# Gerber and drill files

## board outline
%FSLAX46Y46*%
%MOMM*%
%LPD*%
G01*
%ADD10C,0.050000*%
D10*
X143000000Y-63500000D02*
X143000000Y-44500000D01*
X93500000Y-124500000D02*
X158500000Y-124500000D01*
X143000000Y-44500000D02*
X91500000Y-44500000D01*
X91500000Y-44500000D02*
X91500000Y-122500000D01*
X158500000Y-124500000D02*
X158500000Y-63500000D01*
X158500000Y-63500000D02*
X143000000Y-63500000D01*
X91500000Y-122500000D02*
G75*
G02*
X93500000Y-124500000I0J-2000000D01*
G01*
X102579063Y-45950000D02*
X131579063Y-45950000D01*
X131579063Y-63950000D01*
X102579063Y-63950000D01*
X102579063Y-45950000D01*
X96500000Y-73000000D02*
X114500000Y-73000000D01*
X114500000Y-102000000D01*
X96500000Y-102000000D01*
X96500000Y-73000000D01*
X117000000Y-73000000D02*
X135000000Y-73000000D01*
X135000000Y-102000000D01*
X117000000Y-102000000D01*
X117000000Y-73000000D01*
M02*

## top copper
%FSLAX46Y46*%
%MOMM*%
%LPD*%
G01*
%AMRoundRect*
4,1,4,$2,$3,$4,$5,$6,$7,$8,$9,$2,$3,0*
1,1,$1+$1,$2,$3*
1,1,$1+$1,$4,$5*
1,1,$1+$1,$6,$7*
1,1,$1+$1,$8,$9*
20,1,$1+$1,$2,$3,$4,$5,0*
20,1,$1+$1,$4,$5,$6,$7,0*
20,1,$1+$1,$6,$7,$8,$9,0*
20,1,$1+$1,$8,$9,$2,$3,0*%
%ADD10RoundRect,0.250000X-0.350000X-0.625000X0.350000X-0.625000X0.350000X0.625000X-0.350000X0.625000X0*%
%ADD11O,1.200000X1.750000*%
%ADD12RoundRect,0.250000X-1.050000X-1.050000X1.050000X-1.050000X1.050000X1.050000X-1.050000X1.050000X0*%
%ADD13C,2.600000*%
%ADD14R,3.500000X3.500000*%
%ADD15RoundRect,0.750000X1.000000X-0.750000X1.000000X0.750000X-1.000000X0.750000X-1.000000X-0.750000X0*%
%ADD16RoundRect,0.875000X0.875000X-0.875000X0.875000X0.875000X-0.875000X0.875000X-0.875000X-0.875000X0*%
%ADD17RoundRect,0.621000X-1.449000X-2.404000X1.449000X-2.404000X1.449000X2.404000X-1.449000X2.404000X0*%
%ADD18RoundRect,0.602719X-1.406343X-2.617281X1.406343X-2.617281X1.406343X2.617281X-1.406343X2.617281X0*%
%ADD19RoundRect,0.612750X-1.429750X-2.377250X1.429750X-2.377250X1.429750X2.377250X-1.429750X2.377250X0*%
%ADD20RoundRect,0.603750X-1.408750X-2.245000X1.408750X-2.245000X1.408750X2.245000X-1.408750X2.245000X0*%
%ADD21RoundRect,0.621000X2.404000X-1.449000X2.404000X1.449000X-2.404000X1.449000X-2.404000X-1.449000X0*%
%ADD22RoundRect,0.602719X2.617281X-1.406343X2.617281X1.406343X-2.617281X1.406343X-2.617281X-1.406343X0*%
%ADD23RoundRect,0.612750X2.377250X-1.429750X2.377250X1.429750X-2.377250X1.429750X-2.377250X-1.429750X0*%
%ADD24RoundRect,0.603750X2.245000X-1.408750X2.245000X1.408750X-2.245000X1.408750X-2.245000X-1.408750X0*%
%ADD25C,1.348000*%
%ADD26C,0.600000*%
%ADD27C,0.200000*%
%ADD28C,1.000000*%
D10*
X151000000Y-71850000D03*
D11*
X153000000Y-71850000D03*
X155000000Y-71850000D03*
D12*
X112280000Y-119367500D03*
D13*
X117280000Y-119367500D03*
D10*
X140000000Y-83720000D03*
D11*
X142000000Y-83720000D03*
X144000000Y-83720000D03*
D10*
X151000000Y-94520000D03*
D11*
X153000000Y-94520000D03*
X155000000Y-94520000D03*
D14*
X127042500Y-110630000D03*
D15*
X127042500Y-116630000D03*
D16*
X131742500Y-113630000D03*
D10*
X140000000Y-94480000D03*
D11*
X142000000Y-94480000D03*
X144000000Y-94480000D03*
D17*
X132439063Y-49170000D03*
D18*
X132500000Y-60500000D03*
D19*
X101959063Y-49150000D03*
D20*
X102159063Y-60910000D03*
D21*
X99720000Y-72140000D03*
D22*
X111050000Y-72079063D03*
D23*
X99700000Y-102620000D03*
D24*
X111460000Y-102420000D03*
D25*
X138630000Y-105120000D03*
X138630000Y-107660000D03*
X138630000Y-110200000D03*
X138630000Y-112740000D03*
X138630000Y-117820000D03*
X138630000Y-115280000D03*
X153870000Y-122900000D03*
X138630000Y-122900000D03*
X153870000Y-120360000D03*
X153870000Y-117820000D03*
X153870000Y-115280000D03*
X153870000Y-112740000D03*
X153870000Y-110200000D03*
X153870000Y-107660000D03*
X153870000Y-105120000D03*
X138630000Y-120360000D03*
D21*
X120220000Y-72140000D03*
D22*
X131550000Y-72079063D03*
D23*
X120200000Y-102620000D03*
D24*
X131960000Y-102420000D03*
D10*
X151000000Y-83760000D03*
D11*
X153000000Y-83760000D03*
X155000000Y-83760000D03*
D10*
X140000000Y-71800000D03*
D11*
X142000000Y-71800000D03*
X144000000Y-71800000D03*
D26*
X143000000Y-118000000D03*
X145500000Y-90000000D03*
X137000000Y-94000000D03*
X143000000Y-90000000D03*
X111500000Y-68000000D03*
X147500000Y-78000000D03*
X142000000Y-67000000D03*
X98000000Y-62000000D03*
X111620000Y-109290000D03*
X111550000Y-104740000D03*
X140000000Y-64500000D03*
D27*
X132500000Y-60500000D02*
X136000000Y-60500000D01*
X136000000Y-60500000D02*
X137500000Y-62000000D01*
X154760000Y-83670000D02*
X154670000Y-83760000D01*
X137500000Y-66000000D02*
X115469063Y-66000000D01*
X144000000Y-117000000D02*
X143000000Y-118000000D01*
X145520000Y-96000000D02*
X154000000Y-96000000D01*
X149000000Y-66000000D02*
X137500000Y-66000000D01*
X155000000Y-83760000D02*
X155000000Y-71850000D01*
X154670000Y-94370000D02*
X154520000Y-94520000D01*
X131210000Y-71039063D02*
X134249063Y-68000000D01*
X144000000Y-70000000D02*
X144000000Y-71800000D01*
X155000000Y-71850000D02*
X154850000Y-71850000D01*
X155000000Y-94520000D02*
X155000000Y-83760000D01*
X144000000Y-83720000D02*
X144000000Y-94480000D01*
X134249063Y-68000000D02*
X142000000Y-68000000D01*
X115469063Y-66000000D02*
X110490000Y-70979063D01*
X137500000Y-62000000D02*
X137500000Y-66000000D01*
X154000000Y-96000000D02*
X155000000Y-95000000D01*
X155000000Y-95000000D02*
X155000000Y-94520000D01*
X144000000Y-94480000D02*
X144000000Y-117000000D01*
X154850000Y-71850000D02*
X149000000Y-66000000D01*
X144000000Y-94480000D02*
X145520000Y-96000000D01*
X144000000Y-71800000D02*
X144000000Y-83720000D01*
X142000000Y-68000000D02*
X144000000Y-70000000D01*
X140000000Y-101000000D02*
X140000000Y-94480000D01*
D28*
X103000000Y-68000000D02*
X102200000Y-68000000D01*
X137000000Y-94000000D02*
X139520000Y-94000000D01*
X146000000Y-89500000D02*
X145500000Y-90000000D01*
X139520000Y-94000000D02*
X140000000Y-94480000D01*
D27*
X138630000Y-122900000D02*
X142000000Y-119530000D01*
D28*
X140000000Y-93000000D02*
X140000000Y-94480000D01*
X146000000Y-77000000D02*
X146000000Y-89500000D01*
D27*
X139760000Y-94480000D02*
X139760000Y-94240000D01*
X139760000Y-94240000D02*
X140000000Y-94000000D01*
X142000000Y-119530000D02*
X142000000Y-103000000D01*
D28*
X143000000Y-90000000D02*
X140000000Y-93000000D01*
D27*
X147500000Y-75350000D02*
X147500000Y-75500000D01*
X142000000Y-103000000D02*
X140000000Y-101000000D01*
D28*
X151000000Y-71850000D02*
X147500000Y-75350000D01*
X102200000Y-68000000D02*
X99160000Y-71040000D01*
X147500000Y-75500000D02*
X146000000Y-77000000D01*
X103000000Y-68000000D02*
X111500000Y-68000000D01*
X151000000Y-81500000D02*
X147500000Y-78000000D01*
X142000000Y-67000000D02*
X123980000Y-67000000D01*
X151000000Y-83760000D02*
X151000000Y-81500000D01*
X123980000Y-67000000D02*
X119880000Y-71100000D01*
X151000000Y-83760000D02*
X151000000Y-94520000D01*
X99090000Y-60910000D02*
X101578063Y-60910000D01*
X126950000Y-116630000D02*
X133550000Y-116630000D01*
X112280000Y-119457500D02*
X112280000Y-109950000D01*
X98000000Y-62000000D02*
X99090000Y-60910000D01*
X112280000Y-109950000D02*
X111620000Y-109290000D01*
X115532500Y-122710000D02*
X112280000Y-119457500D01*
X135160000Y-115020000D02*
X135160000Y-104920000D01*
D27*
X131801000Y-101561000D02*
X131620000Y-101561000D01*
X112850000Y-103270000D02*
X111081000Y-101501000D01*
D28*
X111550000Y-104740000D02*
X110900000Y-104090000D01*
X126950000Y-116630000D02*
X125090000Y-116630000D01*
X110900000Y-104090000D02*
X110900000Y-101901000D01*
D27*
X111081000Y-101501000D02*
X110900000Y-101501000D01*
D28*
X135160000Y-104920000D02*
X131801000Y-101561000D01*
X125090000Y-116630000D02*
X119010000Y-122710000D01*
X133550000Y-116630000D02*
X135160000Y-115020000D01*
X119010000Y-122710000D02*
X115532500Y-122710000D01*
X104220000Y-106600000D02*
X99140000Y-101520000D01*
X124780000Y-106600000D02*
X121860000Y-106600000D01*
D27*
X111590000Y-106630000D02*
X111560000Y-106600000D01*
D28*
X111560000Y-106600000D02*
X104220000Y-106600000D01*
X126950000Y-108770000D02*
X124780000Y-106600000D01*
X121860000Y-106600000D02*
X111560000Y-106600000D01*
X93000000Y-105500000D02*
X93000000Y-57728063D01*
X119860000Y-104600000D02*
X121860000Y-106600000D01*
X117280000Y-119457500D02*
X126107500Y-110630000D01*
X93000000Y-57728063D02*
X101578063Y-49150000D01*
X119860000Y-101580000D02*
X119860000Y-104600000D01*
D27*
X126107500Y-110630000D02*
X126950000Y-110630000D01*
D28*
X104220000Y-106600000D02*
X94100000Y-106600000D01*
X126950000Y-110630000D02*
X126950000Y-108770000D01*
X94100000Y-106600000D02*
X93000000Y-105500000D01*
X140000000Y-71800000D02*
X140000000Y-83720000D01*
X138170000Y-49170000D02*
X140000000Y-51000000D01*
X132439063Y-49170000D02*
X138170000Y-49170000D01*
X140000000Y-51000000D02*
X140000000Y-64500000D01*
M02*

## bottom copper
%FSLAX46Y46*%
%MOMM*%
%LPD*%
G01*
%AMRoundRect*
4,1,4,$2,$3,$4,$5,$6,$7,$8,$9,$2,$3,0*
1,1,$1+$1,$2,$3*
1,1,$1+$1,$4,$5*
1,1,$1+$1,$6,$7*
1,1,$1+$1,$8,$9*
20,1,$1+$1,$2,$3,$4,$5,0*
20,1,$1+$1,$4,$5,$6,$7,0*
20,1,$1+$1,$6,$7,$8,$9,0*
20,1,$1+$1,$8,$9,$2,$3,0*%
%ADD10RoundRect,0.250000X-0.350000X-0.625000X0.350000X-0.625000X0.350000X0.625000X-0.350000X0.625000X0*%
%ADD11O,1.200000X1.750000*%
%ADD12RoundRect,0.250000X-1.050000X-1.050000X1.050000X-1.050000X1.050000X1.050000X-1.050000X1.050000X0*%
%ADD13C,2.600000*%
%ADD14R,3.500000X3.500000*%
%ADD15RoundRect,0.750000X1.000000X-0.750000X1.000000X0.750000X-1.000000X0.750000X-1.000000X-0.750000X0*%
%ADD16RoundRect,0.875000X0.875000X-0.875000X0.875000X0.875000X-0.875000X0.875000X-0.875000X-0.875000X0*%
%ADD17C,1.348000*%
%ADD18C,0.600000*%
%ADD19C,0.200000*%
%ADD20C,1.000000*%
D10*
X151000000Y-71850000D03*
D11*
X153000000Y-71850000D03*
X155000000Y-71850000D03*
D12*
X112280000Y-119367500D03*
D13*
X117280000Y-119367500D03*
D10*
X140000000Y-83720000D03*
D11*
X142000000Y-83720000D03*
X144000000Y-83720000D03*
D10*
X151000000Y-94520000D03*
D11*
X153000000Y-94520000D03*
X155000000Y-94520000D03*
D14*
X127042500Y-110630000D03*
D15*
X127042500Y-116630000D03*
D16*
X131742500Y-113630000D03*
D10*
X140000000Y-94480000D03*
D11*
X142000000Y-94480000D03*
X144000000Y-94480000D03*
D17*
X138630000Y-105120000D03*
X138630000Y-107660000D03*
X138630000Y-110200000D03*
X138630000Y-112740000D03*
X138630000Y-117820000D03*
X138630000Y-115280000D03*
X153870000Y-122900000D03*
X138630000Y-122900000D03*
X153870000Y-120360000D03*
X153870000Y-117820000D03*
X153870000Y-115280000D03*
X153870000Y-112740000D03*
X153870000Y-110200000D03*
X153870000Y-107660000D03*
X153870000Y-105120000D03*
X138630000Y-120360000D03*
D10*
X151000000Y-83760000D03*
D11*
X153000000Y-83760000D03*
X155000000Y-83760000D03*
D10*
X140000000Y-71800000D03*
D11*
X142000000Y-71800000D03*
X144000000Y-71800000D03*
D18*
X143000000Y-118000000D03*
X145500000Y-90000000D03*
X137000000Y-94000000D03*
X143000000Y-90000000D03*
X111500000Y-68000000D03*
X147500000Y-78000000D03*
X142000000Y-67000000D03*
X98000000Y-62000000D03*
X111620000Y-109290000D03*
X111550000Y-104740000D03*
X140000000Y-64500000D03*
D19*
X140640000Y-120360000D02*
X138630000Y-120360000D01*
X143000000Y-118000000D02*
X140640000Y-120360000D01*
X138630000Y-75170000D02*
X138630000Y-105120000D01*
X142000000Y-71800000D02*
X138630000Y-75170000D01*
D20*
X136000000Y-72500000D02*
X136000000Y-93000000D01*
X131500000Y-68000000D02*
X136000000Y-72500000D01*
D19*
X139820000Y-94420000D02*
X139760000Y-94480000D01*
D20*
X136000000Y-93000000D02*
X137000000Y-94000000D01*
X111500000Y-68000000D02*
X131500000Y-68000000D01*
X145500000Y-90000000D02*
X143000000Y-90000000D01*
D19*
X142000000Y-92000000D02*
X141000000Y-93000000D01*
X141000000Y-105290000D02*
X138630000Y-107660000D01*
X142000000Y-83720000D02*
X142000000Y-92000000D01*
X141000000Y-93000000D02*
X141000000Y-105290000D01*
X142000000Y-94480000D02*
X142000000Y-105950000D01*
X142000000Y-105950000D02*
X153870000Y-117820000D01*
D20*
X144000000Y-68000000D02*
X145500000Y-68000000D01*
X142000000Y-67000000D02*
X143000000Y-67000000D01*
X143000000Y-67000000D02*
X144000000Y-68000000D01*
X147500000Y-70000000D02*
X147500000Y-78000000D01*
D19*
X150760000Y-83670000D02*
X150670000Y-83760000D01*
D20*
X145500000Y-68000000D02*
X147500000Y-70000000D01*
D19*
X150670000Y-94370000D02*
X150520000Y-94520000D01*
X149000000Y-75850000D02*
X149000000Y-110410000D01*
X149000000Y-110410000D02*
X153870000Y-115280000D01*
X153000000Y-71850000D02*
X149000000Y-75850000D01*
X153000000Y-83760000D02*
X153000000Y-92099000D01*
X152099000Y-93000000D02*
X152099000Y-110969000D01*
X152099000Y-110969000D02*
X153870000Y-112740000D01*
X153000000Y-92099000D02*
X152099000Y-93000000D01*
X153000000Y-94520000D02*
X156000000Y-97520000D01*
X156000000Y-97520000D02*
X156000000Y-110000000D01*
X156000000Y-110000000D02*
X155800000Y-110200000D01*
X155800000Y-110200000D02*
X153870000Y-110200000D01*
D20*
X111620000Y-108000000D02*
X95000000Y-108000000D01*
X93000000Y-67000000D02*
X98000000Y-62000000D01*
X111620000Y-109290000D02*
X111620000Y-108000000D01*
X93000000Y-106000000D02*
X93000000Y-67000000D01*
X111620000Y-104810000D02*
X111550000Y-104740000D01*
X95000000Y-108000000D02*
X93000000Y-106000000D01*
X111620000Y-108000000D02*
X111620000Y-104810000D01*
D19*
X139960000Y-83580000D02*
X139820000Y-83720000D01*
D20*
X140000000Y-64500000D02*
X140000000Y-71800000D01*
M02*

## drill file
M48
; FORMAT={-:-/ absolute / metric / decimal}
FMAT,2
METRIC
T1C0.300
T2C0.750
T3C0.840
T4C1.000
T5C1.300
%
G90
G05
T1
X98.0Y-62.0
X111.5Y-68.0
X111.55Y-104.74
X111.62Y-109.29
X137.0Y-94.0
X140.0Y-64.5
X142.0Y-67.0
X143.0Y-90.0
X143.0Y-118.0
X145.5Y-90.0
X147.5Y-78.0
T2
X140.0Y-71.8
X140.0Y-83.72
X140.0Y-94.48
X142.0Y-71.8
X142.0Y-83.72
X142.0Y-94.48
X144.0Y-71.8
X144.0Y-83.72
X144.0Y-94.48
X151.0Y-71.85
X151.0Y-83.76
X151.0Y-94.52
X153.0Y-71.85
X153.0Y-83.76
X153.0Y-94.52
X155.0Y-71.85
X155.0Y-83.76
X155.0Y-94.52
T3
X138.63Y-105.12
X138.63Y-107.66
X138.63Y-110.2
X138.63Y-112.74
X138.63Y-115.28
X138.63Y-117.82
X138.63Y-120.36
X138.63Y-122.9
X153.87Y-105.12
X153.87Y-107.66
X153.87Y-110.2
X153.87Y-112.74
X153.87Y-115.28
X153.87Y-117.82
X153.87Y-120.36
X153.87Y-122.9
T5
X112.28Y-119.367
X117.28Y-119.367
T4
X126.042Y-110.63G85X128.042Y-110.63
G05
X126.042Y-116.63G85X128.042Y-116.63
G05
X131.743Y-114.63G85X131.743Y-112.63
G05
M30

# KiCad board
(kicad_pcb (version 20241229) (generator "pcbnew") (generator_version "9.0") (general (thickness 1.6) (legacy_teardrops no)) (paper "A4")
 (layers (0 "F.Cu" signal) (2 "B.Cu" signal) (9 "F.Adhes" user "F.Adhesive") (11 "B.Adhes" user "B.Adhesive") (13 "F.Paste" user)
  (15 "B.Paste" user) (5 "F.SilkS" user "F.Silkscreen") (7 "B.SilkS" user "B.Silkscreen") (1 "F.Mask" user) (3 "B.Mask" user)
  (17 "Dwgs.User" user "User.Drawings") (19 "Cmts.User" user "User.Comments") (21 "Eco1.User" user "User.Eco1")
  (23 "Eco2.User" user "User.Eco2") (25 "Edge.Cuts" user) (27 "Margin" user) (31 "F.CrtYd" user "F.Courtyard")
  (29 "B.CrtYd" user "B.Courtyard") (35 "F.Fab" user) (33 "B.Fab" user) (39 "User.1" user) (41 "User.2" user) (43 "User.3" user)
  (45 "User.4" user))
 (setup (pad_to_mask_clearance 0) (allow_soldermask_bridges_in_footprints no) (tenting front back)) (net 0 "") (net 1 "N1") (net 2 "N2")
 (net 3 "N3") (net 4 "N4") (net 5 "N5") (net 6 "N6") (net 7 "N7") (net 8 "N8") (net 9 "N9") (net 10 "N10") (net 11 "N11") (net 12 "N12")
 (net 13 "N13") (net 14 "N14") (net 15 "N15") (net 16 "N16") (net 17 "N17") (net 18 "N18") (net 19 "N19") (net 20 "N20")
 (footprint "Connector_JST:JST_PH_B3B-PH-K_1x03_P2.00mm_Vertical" (layer "F.Cu") (at 151 71.85)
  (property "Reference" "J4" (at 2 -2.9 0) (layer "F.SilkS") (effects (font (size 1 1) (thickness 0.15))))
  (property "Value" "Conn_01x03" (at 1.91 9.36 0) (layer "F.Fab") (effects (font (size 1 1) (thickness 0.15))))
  (pad "1" thru_hole roundrect (at 0 0) (size 1.2 1.75) (drill 0.75) (layers "*.Cu" "*.Mask") (remove_unused_layers no)
   (roundrect_rratio 0.208333) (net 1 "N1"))
  (pad "2" thru_hole oval (at 2 0) (size 1.2 1.75) (drill 0.75) (layers "*.Cu" "*.Mask") (remove_unused_layers no) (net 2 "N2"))
  (pad "3" thru_hole oval (at 4 0) (size 1.2 1.75) (drill 0.75) (layers "*.Cu" "*.Mask") (remove_unused_layers no) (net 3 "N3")))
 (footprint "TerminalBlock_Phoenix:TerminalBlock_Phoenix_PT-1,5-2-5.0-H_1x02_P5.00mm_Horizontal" (layer "F.Cu") (at 112.28 119.3675)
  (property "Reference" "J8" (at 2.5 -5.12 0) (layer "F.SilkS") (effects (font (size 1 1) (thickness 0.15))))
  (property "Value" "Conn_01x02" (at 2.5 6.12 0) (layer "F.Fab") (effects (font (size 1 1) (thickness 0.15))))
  (pad "1" thru_hole roundrect (at 0 0) (size 2.6 2.6) (drill 1.3) (layers "*.Cu" "*.Mask") (remove_unused_layers no)
   (roundrect_rratio 0.096154) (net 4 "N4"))
  (pad "2" thru_hole circle (at 5 0) (size 2.6 2.6) (drill 1.3) (layers "*.Cu" "*.Mask") (remove_unused_layers no) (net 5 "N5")))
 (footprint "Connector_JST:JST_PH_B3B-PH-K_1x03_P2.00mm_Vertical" (layer "F.Cu") (at 140 83.72)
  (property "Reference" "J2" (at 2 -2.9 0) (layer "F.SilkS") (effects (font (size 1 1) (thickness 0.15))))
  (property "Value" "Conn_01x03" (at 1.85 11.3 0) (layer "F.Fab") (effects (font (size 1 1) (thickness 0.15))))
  (pad "1" thru_hole roundrect (at 0 0) (size 1.2 1.75) (drill 0.75) (layers "*.Cu" "*.Mask") (remove_unused_layers no)
   (roundrect_rratio 0.208333) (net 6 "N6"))
  (pad "2" thru_hole oval (at 2 0) (size 1.2 1.75) (drill 0.75) (layers "*.Cu" "*.Mask") (remove_unused_layers no) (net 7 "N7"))
  (pad "3" thru_hole oval (at 4 0) (size 1.2 1.75) (drill 0.75) (layers "*.Cu" "*.Mask") (remove_unused_layers no) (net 3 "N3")))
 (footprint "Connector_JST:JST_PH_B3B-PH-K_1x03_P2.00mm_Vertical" (layer "F.Cu") (at 151 94.52)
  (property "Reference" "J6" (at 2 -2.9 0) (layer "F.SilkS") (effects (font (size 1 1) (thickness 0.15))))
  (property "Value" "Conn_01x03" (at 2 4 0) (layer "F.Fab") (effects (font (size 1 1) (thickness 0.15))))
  (pad "1" thru_hole roundrect (at 0 0) (size 1.2 1.75) (drill 0.75) (layers "*.Cu" "*.Mask") (remove_unused_layers no)
   (roundrect_rratio 0.208333) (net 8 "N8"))
  (pad "2" thru_hole oval (at 2 0) (size 1.2 1.75) (drill 0.75) (layers "*.Cu" "*.Mask") (remove_unused_layers no) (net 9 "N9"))
  (pad "3" thru_hole oval (at 4 0) (size 1.2 1.75) (drill 0.75) (layers "*.Cu" "*.Mask") (remove_unused_layers no) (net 3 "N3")))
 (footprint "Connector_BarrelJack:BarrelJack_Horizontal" (layer "F.Cu") (at 127.0425 110.63 90)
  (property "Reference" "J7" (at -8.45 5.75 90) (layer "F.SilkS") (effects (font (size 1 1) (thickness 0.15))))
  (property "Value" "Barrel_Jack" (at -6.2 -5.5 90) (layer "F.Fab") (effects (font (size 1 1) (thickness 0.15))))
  (pad "1" thru_hole rect (at 0 0 90) (size 3.5 3.5) (drill oval 1 3) (layers "*.Cu" "*.Mask") (remove_unused_layers no) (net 5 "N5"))
  (pad "2" thru_hole roundrect (at -6 0 90) (size 3 3.5) (drill oval 1 3) (layers "*.Cu" "*.Mask") (remove_unused_layers no)
   (roundrect_rratio 0.25) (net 4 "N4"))
  (pad "3" thru_hole roundrect (at -3 4.7 90) (size 3.5 3.5) (drill oval 3 1) (layers "*.Cu" "*.Mask") (remove_unused_layers no)
   (roundrect_rratio 0.25)))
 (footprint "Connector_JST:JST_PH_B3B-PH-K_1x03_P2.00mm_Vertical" (layer "F.Cu") (at 140 94.48)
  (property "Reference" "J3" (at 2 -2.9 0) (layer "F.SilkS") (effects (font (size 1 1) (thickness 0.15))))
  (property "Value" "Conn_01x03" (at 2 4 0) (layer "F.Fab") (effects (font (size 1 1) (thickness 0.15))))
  (pad "1" thru_hole roundrect (at 0 0) (size 1.2 1.75) (drill 0.75) (layers "*.Cu" "*.Mask") (remove_unused_layers no)
   (roundrect_rratio 0.208333) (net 1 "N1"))
  (pad "2" thru_hole oval (at 2 0) (size 1.2 1.75) (drill 0.75) (layers "*.Cu" "*.Mask") (remove_unused_layers no) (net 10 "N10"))
  (pad "3" thru_hole oval (at 4 0) (size 1.2 1.75) (drill 0.75) (layers "*.Cu" "*.Mask") (remove_unused_layers no) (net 3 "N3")))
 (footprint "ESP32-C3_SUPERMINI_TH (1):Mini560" (layer "F.Cu") (at 116.579063 52.95)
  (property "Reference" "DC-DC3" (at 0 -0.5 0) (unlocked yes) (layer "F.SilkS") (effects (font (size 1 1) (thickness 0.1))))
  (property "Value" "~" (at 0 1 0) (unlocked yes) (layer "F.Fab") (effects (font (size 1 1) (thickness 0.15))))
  (fp_rect (start -14 -7) (end 15 11) (stroke (width 0.05) (type default)) (fill no) (layer "Edge.Cuts"))
  (pad "1" smd roundrect (at 15.86 -3.78) (size 4.14 6.05) (layers "F.Cu" "F.Mask" "F.Paste") (roundrect_rratio 0.15) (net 6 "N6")
   (thermal_bridge_angle 45))
  (pad "2" smd roundrect (at 15.920937 7.55) (size 4.018125 6.44) (layers "F.Cu" "F.Mask" "F.Paste") (roundrect_rratio 0.15) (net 3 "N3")
   (thermal_bridge_angle 45))
  (pad "3" smd roundrect (at -14.62 -3.8) (size 4.085 5.98) (layers "F.Cu" "F.Mask" "F.Paste") (roundrect_rratio 0.15) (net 5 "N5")
   (thermal_bridge_angle 45))
  (pad "4" smd roundrect (at -14.42 7.96) (size 4.025 5.6975) (layers "F.Cu" "F.Mask" "F.Paste") (roundrect_rratio 0.15) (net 4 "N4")
   (thermal_bridge_angle 45)))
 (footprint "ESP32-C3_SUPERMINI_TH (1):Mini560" (layer "F.Cu") (at 103.5 88 90)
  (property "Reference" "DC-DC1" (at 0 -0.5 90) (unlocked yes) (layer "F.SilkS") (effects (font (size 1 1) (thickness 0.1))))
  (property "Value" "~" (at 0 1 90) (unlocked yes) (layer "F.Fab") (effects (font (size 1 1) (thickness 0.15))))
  (fp_rect (start -14 -7) (end 15 11) (stroke (width 0.05) (type default)) (fill no) (layer "Edge.Cuts"))
  (pad "1" smd roundrect (at 15.86 -3.78 90) (size 4.14 6.05) (layers "F.Cu" "F.Mask" "F.Paste") (roundrect_rratio 0.15) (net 1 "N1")
   (thermal_bridge_angle 45))
  (pad "2" smd roundrect (at 15.920937 7.55 90) (size 4.018125 6.44) (layers "F.Cu" "F.Mask" "F.Paste") (roundrect_rratio 0.15) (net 3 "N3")
   (thermal_bridge_angle 45))
  (pad "3" smd roundrect (at -14.62 -3.8 90) (size 4.085 5.98) (layers "F.Cu" "F.Mask" "F.Paste") (roundrect_rratio 0.15) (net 5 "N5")
   (thermal_bridge_angle 45))
  (pad "4" smd roundrect (at -14.42 7.96 90) (size 4.025 5.6975) (layers "F.Cu" "F.Mask" "F.Paste") (roundrect_rratio 0.15) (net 4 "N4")
   (thermal_bridge_angle 45)))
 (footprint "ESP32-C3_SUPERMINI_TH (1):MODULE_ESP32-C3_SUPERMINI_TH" (layer "F.Cu") (at 146.25 113 180)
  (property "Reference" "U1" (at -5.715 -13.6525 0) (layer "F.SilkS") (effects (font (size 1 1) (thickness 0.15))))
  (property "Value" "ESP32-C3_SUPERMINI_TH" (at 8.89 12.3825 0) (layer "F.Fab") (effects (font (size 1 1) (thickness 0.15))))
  (pad "0" thru_hole circle (at 7.62 7.88 180) (size 1.348 1.348) (drill 0.84) (layers "*.Cu" "*.Mask") (remove_unused_layers no)
   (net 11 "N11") (solder_mask_margin 0.102))
  (pad "1" thru_hole circle (at 7.62 5.34 180) (size 1.348 1.348) (drill 0.84) (layers "*.Cu" "*.Mask") (remove_unused_layers no)
   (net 7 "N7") (solder_mask_margin 0.102))
  (pad "2" thru_hole circle (at 7.62 2.8 180) (size 1.348 1.348) (drill 0.84) (layers "*.Cu" "*.Mask") (remove_unused_layers no)
   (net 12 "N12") (solder_mask_margin 0.102))
  (pad "3" thru_hole circle (at 7.62 0.26 180) (size 1.348 1.348) (drill 0.84) (layers "*.Cu" "*.Mask") (remove_unused_layers no)
   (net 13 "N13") (solder_mask_margin 0.102))
  (pad "3.3" thru_hole circle (at 7.62 -4.82 180) (size 1.348 1.348) (drill 0.84) (layers "*.Cu" "*.Mask") (remove_unused_layers no)
   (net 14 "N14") (solder_mask_margin 0.102))
  (pad "4" thru_hole circle (at 7.62 -2.28 180) (size 1.348 1.348) (drill 0.84) (layers "*.Cu" "*.Mask") (remove_unused_layers no)
   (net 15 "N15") (solder_mask_margin 0.102))
  (pad "5" thru_hole circle (at -7.62 -9.9 180) (size 1.348 1.348) (drill 0.84) (layers "*.Cu" "*.Mask") (remove_unused_layers no)
   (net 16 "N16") (solder_mask_margin 0.102))
  (pad "5V" thru_hole circle (at 7.62 -9.9 180) (size 1.348 1.348) (drill 0.84) (layers "*.Cu" "*.Mask") (remove_unused_layers no)
   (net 1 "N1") (solder_mask_margin 0.102))
  (pad "6" thru_hole circle (at -7.62 -7.36 180) (size 1.348 1.348) (drill 0.84) (layers "*.Cu" "*.Mask") (remove_unused_layers no)
   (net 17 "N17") (solder_mask_margin 0.102))
  (pad "7" thru_hole circle (at -7.62 -4.82 180) (size 1.348 1.348) (drill 0.84) (layers "*.Cu" "*.Mask") (remove_unused_layers no)
   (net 10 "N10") (solder_mask_margin 0.102))
  (pad "8" thru_hole circle (at -7.62 -2.28 180) (size 1.348 1.348) (drill 0.84) (layers "*.Cu" "*.Mask") (remove_unused_layers no)
   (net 2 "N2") (solder_mask_margin 0.102))
  (pad "9" thru_hole circle (at -7.62 0.26 180) (size 1.348 1.348) (drill 0.84) (layers "*.Cu" "*.Mask") (remove_unused_layers no)
   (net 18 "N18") (solder_mask_margin 0.102))
  (pad "10" thru_hole circle (at -7.62 2.8 180) (size 1.348 1.348) (drill 0.84) (layers "*.Cu" "*.Mask") (remove_unused_layers no)
   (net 9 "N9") (solder_mask_margin 0.102))
  (pad "20" thru_hole circle (at -7.62 5.34 180) (size 1.348 1.348) (drill 0.84) (layers "*.Cu" "*.Mask") (remove_unused_layers no)
   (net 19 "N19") (solder_mask_margin 0.102))
  (pad "21" thru_hole circle (at -7.62 7.88 180) (size 1.348 1.348) (drill 0.84) (layers "*.Cu" "*.Mask") (remove_unused_layers no)
   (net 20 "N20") (solder_mask_margin 0.102))
  (pad "G" thru_hole circle (at 7.62 -7.36 180) (size 1.348 1.348) (drill 0.84) (layers "*.Cu" "*.Mask") (remove_unused_layers no)
   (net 3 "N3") (solder_mask_margin 0.102)))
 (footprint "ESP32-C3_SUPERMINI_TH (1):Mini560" (layer "F.Cu") (at 124 88 90)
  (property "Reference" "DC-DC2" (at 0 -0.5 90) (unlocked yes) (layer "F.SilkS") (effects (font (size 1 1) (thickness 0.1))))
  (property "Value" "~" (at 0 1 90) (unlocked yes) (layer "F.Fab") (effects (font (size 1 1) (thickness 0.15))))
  (fp_rect (start -14 -7) (end 15 11) (stroke (width 0.05) (type default)) (fill no) (layer "Edge.Cuts"))
  (pad "1" smd roundrect (at 15.86 -3.78 90) (size 4.14 6.05) (layers "F.Cu" "F.Mask" "F.Paste") (roundrect_rratio 0.15) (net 8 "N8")
   (thermal_bridge_angle 45))
  (pad "2" smd roundrect (at 15.920937 7.55 90) (size 4.018125 6.44) (layers "F.Cu" "F.Mask" "F.Paste") (roundrect_rratio 0.15) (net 3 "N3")
   (thermal_bridge_angle 45))
  (pad "3" smd roundrect (at -14.62 -3.8 90) (size 4.085 5.98) (layers "F.Cu" "F.Mask" "F.Paste") (roundrect_rratio 0.15) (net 5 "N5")
   (thermal_bridge_angle 45))
  (pad "4" smd roundrect (at -14.42 7.96 90) (size 4.025 5.6975) (layers "F.Cu" "F.Mask" "F.Paste") (roundrect_rratio 0.15) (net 4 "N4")
   (thermal_bridge_angle 45)))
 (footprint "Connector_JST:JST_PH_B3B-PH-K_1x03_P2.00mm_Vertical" (layer "F.Cu") (at 151 83.76)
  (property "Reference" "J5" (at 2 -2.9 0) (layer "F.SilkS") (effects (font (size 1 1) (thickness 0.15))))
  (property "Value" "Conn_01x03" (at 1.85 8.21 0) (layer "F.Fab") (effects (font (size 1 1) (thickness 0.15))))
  (pad "1" thru_hole roundrect (at 0 0) (size 1.2 1.75) (drill 0.75) (layers "*.Cu" "*.Mask") (remove_unused_layers no)
   (roundrect_rratio 0.208333) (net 8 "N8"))
  (pad "2" thru_hole oval (at 2 0) (size 1.2 1.75) (drill 0.75) (layers "*.Cu" "*.Mask") (remove_unused_layers no) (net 18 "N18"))
  (pad "3" thru_hole oval (at 4 0) (size 1.2 1.75) (drill 0.75) (layers "*.Cu" "*.Mask") (remove_unused_layers no) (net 3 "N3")))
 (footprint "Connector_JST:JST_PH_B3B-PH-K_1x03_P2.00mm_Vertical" (layer "F.Cu") (at 140 71.8)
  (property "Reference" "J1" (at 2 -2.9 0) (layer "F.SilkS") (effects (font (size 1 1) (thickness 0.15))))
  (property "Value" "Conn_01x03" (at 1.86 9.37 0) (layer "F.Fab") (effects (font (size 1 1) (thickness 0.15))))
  (pad "1" thru_hole roundrect (at 0 0) (size 1.2 1.75) (drill 0.75) (layers "*.Cu" "*.Mask") (remove_unused_layers no)
   (roundrect_rratio 0.208333) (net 6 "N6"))
  (pad "2" thru_hole oval (at 2 0) (size 1.2 1.75) (drill 0.75) (layers "*.Cu" "*.Mask") (remove_unused_layers no) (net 11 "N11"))
  (pad "3" thru_hole oval (at 4 0) (size 1.2 1.75) (drill 0.75) (layers "*.Cu" "*.Mask") (remove_unused_layers no) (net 3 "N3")))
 (gr_line (start 143 63.5) (end 143 44.5) (stroke (width 0.05) (type default)) (layer "Edge.Cuts"))
 (gr_line (start 93.5 124.5) (end 158.5 124.5) (stroke (width 0.05) (type default)) (layer "Edge.Cuts"))
 (gr_line (start 143 44.5) (end 91.5 44.5) (stroke (width 0.05) (type default)) (layer "Edge.Cuts"))
 (gr_line (start 91.5 44.5) (end 91.5 122.5) (stroke (width 0.05) (type default)) (layer "Edge.Cuts"))
 (gr_line (start 158.5 124.5) (end 158.5 63.5) (stroke (width 0.05) (type default)) (layer "Edge.Cuts"))
 (gr_line (start 158.5 63.5) (end 143 63.5) (stroke (width 0.05) (type default)) (layer "Edge.Cuts"))
 (gr_arc (start 91.5 122.5) (mid 92.914214 123.085786) (end 93.5 124.5) (stroke (width 0.05) (type default)) (layer "Edge.Cuts"))
 (segment (start 132.5 60.5) (end 136 60.5) (width 0.2) (layer "F.Cu") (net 3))
 (segment (start 136 60.5) (end 137.5 62) (width 0.2) (layer "F.Cu") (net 3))
 (segment (start 154.76 83.67) (end 154.67 83.76) (width 0.2) (layer "F.Cu") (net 3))
 (segment (start 137.5 66) (end 115.469063 66) (width 0.2) (layer "F.Cu") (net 3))
 (segment (start 144 117) (end 143 118) (width 0.2) (layer "F.Cu") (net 3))
 (segment (start 145.52 96) (end 154 96) (width 0.2) (layer "F.Cu") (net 3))
 (segment (start 149 66) (end 137.5 66) (width 0.2) (layer "F.Cu") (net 3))
 (segment (start 155 83.76) (end 155 71.85) (width 0.2) (layer "F.Cu") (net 3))
 (segment (start 154.67 94.37) (end 154.52 94.52) (width 0.2) (layer "F.Cu") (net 3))
 (segment (start 131.21 71.039063) (end 134.249063 68) (width 0.2) (layer "F.Cu") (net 3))
 (segment (start 144 70) (end 144 71.8) (width 0.2) (layer "F.Cu") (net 3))
 (segment (start 155 71.85) (end 154.85 71.85) (width 0.2) (layer "F.Cu") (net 3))
 (segment (start 155 94.52) (end 155 83.76) (width 0.2) (layer "F.Cu") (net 3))
 (segment (start 144 83.72) (end 144 94.48) (width 0.2) (layer "F.Cu") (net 3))
 (segment (start 134.249063 68) (end 142 68) (width 0.2) (layer "F.Cu") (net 3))
 (segment (start 115.469063 66) (end 110.49 70.979063) (width 0.2) (layer "F.Cu") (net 3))
 (segment (start 137.5 62) (end 137.5 66) (width 0.2) (layer "F.Cu") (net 3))
 (segment (start 154 96) (end 155 95) (width 0.2) (layer "F.Cu") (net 3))
 (segment (start 155 95) (end 155 94.52) (width 0.2) (layer "F.Cu") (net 3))
 (segment (start 144 94.48) (end 144 117) (width 0.2) (layer "F.Cu") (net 3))
 (segment (start 154.85 71.85) (end 149 66) (width 0.2) (layer "F.Cu") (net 3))
 (segment (start 144 94.48) (end 145.52 96) (width 0.2) (layer "F.Cu") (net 3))
 (segment (start 144 71.8) (end 144 83.72) (width 0.2) (layer "F.Cu") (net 3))
 (segment (start 142 68) (end 144 70) (width 0.2) (layer "F.Cu") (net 3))
 (via (at 143 118) (size 0.6) (drill 0.3) (layers "F.Cu" "B.Cu") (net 3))
 (segment (start 140.64 120.36) (end 138.63 120.36) (width 0.2) (layer "B.Cu") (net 3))
 (segment (start 143 118) (end 140.64 120.36) (width 0.2) (layer "B.Cu") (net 3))
 (segment (start 138.63 75.17) (end 138.63 105.12) (width 0.2) (layer "B.Cu") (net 11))
 (segment (start 142 71.8) (end 138.63 75.17) (width 0.2) (layer "B.Cu") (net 11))
 (segment (start 140 101) (end 140 94.48) (width 0.2) (layer "F.Cu") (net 1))
 (segment (start 103 68) (end 102.2 68) (width 1) (layer "F.Cu") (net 1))
 (segment (start 137 94) (end 139.52 94) (width 1) (layer "F.Cu") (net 1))
 (segment (start 146 89.5) (end 145.5 90) (width 1) (layer "F.Cu") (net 1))
 (segment (start 139.52 94) (end 140 94.48) (width 1) (layer "F.Cu") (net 1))
 (segment (start 138.63 122.9) (end 142 119.53) (width 0.2) (layer "F.Cu") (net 1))
 (segment (start 140 93) (end 140 94.48) (width 1) (layer "F.Cu") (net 1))
 (segment (start 146 77) (end 146 89.5) (width 1) (layer "F.Cu") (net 1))
 (segment (start 139.76 94.48) (end 139.76 94.24) (width 0.2) (layer "F.Cu") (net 1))
 (segment (start 139.76 94.24) (end 140 94) (width 0.2) (layer "F.Cu") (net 1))
 (segment (start 142 119.53) (end 142 103) (width 0.2) (layer "F.Cu") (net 1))
 (segment (start 143 90) (end 140 93) (width 1) (layer "F.Cu") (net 1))
 (segment (start 147.5 75.35) (end 147.5 75.5) (width 0.2) (layer "F.Cu") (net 1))
 (segment (start 142 103) (end 140 101) (width 0.2) (layer "F.Cu") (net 1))
 (segment (start 151 71.85) (end 147.5 75.35) (width 1) (layer "F.Cu") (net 1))
 (segment (start 102.2 68) (end 99.16 71.04) (width 1) (layer "F.Cu") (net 1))
 (segment (start 147.5 75.5) (end 146 77) (width 1) (layer "F.Cu") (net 1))
 (segment (start 103 68) (end 111.5 68) (width 1) (layer "F.Cu") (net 1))
 (via (at 145.5 90) (size 0.6) (drill 0.3) (layers "F.Cu" "B.Cu") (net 1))
 (via (at 137 94) (size 0.6) (drill 0.3) (layers "F.Cu" "B.Cu") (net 1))
 (via (at 143 90) (size 0.6) (drill 0.3) (layers "F.Cu" "B.Cu") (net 1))
 (via (at 111.5 68) (size 0.6) (drill 0.3) (layers "F.Cu" "B.Cu") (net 1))
 (segment (start 136 72.5) (end 136 93) (width 1) (layer "B.Cu") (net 1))
 (segment (start 131.5 68) (end 136 72.5) (width 1) (layer "B.Cu") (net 1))
 (segment (start 139.82 94.42) (end 139.76 94.48) (width 0.2) (layer "B.Cu") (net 1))
 (segment (start 136 93) (end 137 94) (width 1) (layer "B.Cu") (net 1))
 (segment (start 111.5 68) (end 131.5 68) (width 1) (layer "B.Cu") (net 1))
 (segment (start 145.5 90) (end 143 90) (width 1) (layer "B.Cu") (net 1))
 (segment (start 142 92) (end 141 93) (width 0.2) (layer "B.Cu") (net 7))
 (segment (start 141 105.29) (end 138.63 107.66) (width 0.2) (layer "B.Cu") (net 7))
 (segment (start 142 83.72) (end 142 92) (width 0.2) (layer "B.Cu") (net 7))
 (segment (start 141 93) (end 141 105.29) (width 0.2) (layer "B.Cu") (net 7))
 (segment (start 142 94.48) (end 142 105.95) (width 0.2) (layer "B.Cu") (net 10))
 (segment (start 142 105.95) (end 153.87 117.82) (width 0.2) (layer "B.Cu") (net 10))
 (segment (start 151 81.5) (end 147.5 78) (width 1) (layer "F.Cu") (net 8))
 (segment (start 142 67) (end 123.98 67) (width 1) (layer "F.Cu") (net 8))
 (segment (start 151 83.76) (end 151 81.5) (width 1) (layer "F.Cu") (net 8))
 (segment (start 123.98 67) (end 119.88 71.1) (width 1) (layer "F.Cu") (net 8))
 (segment (start 151 83.76) (end 151 94.52) (width 1) (layer "F.Cu") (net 8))
 (via (at 147.5 78) (size 0.6) (drill 0.3) (layers "F.Cu" "B.Cu") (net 8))
 (via (at 142 67) (size 0.6) (drill 0.3) (layers "F.Cu" "B.Cu") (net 8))
 (segment (start 144 68) (end 145.5 68) (width 1) (layer "B.Cu") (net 8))
 (segment (start 142 67) (end 143 67) (width 1) (layer "B.Cu") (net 8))
 (segment (start 143 67) (end 144 68) (width 1) (layer "B.Cu") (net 8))
 (segment (start 147.5 70) (end 147.5 78) (width 1) (layer "B.Cu") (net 8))
 (segment (start 150.76 83.67) (end 150.67 83.76) (width 0.2) (layer "B.Cu") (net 8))
 (segment (start 145.5 68) (end 147.5 70) (width 1) (layer "B.Cu") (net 8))
 (segment (start 150.67 94.37) (end 150.52 94.52) (width 0.2) (layer "B.Cu") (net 8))
 (segment (start 149 75.85) (end 149 110.41) (width 0.2) (layer "B.Cu") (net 2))
 (segment (start 149 110.41) (end 153.87 115.28) (width 0.2) (layer "B.Cu") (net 2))
 (segment (start 153 71.85) (end 149 75.85) (width 0.2) (layer "B.Cu") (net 2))
 (segment (start 153 83.76) (end 153 92.099) (width 0.2) (layer "B.Cu") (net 18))
 (segment (start 152.099 93) (end 152.099 110.969) (width 0.2) (layer "B.Cu") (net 18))
 (segment (start 152.099 110.969) (end 153.87 112.74) (width 0.2) (layer "B.Cu") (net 18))
 (segment (start 153 92.099) (end 152.099 93) (width 0.2) (layer "B.Cu") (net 18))
 (segment (start 153 94.52) (end 156 97.52) (width 0.2) (layer "B.Cu") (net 9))
 (segment (start 156 97.52) (end 156 110) (width 0.2) (layer "B.Cu") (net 9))
 (segment (start 156 110) (end 155.8 110.2) (width 0.2) (layer "B.Cu") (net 9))
 (segment (start 155.8 110.2) (end 153.87 110.2) (width 0.2) (layer "B.Cu") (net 9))
 (segment (start 99.09 60.91) (end 101.578063 60.91) (width 1) (layer "F.Cu") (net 4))
 (segment (start 126.95 116.63) (end 133.55 116.63) (width 1) (layer "F.Cu") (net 4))
 (segment (start 112.28 119.4575) (end 112.28 109.95) (width 1) (layer "F.Cu") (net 4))
 (segment (start 98 62) (end 99.09 60.91) (width 1) (layer "F.Cu") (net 4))
 (segment (start 112.28 109.95) (end 111.62 109.29) (width 1) (layer "F.Cu") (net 4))
 (segment (start 115.5325 122.71) (end 112.28 119.4575) (width 1) (layer "F.Cu") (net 4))
 (segment (start 135.16 115.02) (end 135.16 104.92) (width 1) (layer "F.Cu") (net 4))
 (segment (start 131.801 101.561) (end 131.62 101.561) (width 0.2) (layer "F.Cu") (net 4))
 (segment (start 112.85 103.27) (end 111.081 101.501) (width 0.2) (layer "F.Cu") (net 4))
 (segment (start 111.55 104.74) (end 110.9 104.09) (width 1) (layer "F.Cu") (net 4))
 (segment (start 126.95 116.63) (end 125.09 116.63) (width 1) (layer "F.Cu") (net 4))
 (segment (start 110.9 104.09) (end 110.9 101.901) (width 1) (layer "F.Cu") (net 4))
 (segment (start 111.081 101.501) (end 110.9 101.501) (width 0.2) (layer "F.Cu") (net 4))
 (segment (start 135.16 104.92) (end 131.801 101.561) (width 1) (layer "F.Cu") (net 4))
 (segment (start 125.09 116.63) (end 119.01 122.71) (width 1) (layer "F.Cu") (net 4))
 (segment (start 133.55 116.63) (end 135.16 115.02) (width 1) (layer "F.Cu") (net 4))
 (segment (start 119.01 122.71) (end 115.5325 122.71) (width 1) (layer "F.Cu") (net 4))
 (via (at 98 62) (size 0.6) (drill 0.3) (layers "F.Cu" "B.Cu") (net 4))
 (via (at 111.62 109.29) (size 0.6) (drill 0.3) (layers "F.Cu" "B.Cu") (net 4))
 (via (at 111.55 104.74) (size 0.6) (drill 0.3) (layers "F.Cu" "B.Cu") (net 4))
 (segment (start 111.62 108) (end 95 108) (width 1) (layer "B.Cu") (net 4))
 (segment (start 93 67) (end 98 62) (width 1) (layer "B.Cu") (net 4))
 (segment (start 111.62 109.29) (end 111.62 108) (width 1) (layer "B.Cu") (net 4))
 (segment (start 93 106) (end 93 67) (width 1) (layer "B.Cu") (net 4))
 (segment (start 111.62 104.81) (end 111.55 104.74) (width 1) (layer "B.Cu") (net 4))
 (segment (start 95 108) (end 93 106) (width 1) (layer "B.Cu") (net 4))
 (segment (start 111.62 108) (end 111.62 104.81) (width 1) (layer "B.Cu") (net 4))
 (segment (start 104.22 106.6) (end 99.14 101.52) (width 1) (layer "F.Cu") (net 5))
 (segment (start 124.78 106.6) (end 121.86 106.6) (width 1) (layer "F.Cu") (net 5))
 (segment (start 111.59 106.63) (end 111.56 106.6) (width 0.2) (layer "F.Cu") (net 5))
 (segment (start 111.56 106.6) (end 104.22 106.6) (width 1) (layer "F.Cu") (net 5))
 (segment (start 126.95 108.77) (end 124.78 106.6) (width 1) (layer "F.Cu") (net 5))
 (segment (start 121.86 106.6) (end 111.56 106.6) (width 1) (layer "F.Cu") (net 5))
 (segment (start 93 105.5) (end 93 57.728063) (width 1) (layer "F.Cu") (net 5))
 (segment (start 119.86 104.6) (end 121.86 106.6) (width 1) (layer "F.Cu") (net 5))
 (segment (start 117.28 119.4575) (end 126.1075 110.63) (width 1) (layer "F.Cu") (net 5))
 (segment (start 93 57.728063) (end 101.578063 49.15) (width 1) (layer "F.Cu") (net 5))
 (segment (start 119.86 101.58) (end 119.86 104.6) (width 1) (layer "F.Cu") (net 5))
 (segment (start 126.1075 110.63) (end 126.95 110.63) (width 0.2) (layer "F.Cu") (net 5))
 (segment (start 104.22 106.6) (end 94.1 106.6) (width 1) (layer "F.Cu") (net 5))
 (segment (start 126.95 110.63) (end 126.95 108.77) (width 1) (layer "F.Cu") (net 5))
 (segment (start 94.1 106.6) (end 93 105.5) (width 1) (layer "F.Cu") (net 5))
 (segment (start 140 71.8) (end 140 83.72) (width 1) (layer "F.Cu") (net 6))
 (segment (start 138.17 49.17) (end 140 51) (width 1) (layer "F.Cu") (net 6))
 (segment (start 132.439063 49.17) (end 138.17 49.17) (width 1) (layer "F.Cu") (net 6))
 (segment (start 140 51) (end 140 64.5) (width 1) (layer "F.Cu") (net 6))
 (via (at 140 64.5) (size 0.6) (drill 0.3) (layers "F.Cu" "B.Cu") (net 6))
 (segment (start 139.96 83.58) (end 139.82 83.72) (width 0.2) (layer "B.Cu") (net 6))
 (segment (start 140 64.5) (end 140 71.8) (width 1) (layer "B.Cu") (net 6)))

